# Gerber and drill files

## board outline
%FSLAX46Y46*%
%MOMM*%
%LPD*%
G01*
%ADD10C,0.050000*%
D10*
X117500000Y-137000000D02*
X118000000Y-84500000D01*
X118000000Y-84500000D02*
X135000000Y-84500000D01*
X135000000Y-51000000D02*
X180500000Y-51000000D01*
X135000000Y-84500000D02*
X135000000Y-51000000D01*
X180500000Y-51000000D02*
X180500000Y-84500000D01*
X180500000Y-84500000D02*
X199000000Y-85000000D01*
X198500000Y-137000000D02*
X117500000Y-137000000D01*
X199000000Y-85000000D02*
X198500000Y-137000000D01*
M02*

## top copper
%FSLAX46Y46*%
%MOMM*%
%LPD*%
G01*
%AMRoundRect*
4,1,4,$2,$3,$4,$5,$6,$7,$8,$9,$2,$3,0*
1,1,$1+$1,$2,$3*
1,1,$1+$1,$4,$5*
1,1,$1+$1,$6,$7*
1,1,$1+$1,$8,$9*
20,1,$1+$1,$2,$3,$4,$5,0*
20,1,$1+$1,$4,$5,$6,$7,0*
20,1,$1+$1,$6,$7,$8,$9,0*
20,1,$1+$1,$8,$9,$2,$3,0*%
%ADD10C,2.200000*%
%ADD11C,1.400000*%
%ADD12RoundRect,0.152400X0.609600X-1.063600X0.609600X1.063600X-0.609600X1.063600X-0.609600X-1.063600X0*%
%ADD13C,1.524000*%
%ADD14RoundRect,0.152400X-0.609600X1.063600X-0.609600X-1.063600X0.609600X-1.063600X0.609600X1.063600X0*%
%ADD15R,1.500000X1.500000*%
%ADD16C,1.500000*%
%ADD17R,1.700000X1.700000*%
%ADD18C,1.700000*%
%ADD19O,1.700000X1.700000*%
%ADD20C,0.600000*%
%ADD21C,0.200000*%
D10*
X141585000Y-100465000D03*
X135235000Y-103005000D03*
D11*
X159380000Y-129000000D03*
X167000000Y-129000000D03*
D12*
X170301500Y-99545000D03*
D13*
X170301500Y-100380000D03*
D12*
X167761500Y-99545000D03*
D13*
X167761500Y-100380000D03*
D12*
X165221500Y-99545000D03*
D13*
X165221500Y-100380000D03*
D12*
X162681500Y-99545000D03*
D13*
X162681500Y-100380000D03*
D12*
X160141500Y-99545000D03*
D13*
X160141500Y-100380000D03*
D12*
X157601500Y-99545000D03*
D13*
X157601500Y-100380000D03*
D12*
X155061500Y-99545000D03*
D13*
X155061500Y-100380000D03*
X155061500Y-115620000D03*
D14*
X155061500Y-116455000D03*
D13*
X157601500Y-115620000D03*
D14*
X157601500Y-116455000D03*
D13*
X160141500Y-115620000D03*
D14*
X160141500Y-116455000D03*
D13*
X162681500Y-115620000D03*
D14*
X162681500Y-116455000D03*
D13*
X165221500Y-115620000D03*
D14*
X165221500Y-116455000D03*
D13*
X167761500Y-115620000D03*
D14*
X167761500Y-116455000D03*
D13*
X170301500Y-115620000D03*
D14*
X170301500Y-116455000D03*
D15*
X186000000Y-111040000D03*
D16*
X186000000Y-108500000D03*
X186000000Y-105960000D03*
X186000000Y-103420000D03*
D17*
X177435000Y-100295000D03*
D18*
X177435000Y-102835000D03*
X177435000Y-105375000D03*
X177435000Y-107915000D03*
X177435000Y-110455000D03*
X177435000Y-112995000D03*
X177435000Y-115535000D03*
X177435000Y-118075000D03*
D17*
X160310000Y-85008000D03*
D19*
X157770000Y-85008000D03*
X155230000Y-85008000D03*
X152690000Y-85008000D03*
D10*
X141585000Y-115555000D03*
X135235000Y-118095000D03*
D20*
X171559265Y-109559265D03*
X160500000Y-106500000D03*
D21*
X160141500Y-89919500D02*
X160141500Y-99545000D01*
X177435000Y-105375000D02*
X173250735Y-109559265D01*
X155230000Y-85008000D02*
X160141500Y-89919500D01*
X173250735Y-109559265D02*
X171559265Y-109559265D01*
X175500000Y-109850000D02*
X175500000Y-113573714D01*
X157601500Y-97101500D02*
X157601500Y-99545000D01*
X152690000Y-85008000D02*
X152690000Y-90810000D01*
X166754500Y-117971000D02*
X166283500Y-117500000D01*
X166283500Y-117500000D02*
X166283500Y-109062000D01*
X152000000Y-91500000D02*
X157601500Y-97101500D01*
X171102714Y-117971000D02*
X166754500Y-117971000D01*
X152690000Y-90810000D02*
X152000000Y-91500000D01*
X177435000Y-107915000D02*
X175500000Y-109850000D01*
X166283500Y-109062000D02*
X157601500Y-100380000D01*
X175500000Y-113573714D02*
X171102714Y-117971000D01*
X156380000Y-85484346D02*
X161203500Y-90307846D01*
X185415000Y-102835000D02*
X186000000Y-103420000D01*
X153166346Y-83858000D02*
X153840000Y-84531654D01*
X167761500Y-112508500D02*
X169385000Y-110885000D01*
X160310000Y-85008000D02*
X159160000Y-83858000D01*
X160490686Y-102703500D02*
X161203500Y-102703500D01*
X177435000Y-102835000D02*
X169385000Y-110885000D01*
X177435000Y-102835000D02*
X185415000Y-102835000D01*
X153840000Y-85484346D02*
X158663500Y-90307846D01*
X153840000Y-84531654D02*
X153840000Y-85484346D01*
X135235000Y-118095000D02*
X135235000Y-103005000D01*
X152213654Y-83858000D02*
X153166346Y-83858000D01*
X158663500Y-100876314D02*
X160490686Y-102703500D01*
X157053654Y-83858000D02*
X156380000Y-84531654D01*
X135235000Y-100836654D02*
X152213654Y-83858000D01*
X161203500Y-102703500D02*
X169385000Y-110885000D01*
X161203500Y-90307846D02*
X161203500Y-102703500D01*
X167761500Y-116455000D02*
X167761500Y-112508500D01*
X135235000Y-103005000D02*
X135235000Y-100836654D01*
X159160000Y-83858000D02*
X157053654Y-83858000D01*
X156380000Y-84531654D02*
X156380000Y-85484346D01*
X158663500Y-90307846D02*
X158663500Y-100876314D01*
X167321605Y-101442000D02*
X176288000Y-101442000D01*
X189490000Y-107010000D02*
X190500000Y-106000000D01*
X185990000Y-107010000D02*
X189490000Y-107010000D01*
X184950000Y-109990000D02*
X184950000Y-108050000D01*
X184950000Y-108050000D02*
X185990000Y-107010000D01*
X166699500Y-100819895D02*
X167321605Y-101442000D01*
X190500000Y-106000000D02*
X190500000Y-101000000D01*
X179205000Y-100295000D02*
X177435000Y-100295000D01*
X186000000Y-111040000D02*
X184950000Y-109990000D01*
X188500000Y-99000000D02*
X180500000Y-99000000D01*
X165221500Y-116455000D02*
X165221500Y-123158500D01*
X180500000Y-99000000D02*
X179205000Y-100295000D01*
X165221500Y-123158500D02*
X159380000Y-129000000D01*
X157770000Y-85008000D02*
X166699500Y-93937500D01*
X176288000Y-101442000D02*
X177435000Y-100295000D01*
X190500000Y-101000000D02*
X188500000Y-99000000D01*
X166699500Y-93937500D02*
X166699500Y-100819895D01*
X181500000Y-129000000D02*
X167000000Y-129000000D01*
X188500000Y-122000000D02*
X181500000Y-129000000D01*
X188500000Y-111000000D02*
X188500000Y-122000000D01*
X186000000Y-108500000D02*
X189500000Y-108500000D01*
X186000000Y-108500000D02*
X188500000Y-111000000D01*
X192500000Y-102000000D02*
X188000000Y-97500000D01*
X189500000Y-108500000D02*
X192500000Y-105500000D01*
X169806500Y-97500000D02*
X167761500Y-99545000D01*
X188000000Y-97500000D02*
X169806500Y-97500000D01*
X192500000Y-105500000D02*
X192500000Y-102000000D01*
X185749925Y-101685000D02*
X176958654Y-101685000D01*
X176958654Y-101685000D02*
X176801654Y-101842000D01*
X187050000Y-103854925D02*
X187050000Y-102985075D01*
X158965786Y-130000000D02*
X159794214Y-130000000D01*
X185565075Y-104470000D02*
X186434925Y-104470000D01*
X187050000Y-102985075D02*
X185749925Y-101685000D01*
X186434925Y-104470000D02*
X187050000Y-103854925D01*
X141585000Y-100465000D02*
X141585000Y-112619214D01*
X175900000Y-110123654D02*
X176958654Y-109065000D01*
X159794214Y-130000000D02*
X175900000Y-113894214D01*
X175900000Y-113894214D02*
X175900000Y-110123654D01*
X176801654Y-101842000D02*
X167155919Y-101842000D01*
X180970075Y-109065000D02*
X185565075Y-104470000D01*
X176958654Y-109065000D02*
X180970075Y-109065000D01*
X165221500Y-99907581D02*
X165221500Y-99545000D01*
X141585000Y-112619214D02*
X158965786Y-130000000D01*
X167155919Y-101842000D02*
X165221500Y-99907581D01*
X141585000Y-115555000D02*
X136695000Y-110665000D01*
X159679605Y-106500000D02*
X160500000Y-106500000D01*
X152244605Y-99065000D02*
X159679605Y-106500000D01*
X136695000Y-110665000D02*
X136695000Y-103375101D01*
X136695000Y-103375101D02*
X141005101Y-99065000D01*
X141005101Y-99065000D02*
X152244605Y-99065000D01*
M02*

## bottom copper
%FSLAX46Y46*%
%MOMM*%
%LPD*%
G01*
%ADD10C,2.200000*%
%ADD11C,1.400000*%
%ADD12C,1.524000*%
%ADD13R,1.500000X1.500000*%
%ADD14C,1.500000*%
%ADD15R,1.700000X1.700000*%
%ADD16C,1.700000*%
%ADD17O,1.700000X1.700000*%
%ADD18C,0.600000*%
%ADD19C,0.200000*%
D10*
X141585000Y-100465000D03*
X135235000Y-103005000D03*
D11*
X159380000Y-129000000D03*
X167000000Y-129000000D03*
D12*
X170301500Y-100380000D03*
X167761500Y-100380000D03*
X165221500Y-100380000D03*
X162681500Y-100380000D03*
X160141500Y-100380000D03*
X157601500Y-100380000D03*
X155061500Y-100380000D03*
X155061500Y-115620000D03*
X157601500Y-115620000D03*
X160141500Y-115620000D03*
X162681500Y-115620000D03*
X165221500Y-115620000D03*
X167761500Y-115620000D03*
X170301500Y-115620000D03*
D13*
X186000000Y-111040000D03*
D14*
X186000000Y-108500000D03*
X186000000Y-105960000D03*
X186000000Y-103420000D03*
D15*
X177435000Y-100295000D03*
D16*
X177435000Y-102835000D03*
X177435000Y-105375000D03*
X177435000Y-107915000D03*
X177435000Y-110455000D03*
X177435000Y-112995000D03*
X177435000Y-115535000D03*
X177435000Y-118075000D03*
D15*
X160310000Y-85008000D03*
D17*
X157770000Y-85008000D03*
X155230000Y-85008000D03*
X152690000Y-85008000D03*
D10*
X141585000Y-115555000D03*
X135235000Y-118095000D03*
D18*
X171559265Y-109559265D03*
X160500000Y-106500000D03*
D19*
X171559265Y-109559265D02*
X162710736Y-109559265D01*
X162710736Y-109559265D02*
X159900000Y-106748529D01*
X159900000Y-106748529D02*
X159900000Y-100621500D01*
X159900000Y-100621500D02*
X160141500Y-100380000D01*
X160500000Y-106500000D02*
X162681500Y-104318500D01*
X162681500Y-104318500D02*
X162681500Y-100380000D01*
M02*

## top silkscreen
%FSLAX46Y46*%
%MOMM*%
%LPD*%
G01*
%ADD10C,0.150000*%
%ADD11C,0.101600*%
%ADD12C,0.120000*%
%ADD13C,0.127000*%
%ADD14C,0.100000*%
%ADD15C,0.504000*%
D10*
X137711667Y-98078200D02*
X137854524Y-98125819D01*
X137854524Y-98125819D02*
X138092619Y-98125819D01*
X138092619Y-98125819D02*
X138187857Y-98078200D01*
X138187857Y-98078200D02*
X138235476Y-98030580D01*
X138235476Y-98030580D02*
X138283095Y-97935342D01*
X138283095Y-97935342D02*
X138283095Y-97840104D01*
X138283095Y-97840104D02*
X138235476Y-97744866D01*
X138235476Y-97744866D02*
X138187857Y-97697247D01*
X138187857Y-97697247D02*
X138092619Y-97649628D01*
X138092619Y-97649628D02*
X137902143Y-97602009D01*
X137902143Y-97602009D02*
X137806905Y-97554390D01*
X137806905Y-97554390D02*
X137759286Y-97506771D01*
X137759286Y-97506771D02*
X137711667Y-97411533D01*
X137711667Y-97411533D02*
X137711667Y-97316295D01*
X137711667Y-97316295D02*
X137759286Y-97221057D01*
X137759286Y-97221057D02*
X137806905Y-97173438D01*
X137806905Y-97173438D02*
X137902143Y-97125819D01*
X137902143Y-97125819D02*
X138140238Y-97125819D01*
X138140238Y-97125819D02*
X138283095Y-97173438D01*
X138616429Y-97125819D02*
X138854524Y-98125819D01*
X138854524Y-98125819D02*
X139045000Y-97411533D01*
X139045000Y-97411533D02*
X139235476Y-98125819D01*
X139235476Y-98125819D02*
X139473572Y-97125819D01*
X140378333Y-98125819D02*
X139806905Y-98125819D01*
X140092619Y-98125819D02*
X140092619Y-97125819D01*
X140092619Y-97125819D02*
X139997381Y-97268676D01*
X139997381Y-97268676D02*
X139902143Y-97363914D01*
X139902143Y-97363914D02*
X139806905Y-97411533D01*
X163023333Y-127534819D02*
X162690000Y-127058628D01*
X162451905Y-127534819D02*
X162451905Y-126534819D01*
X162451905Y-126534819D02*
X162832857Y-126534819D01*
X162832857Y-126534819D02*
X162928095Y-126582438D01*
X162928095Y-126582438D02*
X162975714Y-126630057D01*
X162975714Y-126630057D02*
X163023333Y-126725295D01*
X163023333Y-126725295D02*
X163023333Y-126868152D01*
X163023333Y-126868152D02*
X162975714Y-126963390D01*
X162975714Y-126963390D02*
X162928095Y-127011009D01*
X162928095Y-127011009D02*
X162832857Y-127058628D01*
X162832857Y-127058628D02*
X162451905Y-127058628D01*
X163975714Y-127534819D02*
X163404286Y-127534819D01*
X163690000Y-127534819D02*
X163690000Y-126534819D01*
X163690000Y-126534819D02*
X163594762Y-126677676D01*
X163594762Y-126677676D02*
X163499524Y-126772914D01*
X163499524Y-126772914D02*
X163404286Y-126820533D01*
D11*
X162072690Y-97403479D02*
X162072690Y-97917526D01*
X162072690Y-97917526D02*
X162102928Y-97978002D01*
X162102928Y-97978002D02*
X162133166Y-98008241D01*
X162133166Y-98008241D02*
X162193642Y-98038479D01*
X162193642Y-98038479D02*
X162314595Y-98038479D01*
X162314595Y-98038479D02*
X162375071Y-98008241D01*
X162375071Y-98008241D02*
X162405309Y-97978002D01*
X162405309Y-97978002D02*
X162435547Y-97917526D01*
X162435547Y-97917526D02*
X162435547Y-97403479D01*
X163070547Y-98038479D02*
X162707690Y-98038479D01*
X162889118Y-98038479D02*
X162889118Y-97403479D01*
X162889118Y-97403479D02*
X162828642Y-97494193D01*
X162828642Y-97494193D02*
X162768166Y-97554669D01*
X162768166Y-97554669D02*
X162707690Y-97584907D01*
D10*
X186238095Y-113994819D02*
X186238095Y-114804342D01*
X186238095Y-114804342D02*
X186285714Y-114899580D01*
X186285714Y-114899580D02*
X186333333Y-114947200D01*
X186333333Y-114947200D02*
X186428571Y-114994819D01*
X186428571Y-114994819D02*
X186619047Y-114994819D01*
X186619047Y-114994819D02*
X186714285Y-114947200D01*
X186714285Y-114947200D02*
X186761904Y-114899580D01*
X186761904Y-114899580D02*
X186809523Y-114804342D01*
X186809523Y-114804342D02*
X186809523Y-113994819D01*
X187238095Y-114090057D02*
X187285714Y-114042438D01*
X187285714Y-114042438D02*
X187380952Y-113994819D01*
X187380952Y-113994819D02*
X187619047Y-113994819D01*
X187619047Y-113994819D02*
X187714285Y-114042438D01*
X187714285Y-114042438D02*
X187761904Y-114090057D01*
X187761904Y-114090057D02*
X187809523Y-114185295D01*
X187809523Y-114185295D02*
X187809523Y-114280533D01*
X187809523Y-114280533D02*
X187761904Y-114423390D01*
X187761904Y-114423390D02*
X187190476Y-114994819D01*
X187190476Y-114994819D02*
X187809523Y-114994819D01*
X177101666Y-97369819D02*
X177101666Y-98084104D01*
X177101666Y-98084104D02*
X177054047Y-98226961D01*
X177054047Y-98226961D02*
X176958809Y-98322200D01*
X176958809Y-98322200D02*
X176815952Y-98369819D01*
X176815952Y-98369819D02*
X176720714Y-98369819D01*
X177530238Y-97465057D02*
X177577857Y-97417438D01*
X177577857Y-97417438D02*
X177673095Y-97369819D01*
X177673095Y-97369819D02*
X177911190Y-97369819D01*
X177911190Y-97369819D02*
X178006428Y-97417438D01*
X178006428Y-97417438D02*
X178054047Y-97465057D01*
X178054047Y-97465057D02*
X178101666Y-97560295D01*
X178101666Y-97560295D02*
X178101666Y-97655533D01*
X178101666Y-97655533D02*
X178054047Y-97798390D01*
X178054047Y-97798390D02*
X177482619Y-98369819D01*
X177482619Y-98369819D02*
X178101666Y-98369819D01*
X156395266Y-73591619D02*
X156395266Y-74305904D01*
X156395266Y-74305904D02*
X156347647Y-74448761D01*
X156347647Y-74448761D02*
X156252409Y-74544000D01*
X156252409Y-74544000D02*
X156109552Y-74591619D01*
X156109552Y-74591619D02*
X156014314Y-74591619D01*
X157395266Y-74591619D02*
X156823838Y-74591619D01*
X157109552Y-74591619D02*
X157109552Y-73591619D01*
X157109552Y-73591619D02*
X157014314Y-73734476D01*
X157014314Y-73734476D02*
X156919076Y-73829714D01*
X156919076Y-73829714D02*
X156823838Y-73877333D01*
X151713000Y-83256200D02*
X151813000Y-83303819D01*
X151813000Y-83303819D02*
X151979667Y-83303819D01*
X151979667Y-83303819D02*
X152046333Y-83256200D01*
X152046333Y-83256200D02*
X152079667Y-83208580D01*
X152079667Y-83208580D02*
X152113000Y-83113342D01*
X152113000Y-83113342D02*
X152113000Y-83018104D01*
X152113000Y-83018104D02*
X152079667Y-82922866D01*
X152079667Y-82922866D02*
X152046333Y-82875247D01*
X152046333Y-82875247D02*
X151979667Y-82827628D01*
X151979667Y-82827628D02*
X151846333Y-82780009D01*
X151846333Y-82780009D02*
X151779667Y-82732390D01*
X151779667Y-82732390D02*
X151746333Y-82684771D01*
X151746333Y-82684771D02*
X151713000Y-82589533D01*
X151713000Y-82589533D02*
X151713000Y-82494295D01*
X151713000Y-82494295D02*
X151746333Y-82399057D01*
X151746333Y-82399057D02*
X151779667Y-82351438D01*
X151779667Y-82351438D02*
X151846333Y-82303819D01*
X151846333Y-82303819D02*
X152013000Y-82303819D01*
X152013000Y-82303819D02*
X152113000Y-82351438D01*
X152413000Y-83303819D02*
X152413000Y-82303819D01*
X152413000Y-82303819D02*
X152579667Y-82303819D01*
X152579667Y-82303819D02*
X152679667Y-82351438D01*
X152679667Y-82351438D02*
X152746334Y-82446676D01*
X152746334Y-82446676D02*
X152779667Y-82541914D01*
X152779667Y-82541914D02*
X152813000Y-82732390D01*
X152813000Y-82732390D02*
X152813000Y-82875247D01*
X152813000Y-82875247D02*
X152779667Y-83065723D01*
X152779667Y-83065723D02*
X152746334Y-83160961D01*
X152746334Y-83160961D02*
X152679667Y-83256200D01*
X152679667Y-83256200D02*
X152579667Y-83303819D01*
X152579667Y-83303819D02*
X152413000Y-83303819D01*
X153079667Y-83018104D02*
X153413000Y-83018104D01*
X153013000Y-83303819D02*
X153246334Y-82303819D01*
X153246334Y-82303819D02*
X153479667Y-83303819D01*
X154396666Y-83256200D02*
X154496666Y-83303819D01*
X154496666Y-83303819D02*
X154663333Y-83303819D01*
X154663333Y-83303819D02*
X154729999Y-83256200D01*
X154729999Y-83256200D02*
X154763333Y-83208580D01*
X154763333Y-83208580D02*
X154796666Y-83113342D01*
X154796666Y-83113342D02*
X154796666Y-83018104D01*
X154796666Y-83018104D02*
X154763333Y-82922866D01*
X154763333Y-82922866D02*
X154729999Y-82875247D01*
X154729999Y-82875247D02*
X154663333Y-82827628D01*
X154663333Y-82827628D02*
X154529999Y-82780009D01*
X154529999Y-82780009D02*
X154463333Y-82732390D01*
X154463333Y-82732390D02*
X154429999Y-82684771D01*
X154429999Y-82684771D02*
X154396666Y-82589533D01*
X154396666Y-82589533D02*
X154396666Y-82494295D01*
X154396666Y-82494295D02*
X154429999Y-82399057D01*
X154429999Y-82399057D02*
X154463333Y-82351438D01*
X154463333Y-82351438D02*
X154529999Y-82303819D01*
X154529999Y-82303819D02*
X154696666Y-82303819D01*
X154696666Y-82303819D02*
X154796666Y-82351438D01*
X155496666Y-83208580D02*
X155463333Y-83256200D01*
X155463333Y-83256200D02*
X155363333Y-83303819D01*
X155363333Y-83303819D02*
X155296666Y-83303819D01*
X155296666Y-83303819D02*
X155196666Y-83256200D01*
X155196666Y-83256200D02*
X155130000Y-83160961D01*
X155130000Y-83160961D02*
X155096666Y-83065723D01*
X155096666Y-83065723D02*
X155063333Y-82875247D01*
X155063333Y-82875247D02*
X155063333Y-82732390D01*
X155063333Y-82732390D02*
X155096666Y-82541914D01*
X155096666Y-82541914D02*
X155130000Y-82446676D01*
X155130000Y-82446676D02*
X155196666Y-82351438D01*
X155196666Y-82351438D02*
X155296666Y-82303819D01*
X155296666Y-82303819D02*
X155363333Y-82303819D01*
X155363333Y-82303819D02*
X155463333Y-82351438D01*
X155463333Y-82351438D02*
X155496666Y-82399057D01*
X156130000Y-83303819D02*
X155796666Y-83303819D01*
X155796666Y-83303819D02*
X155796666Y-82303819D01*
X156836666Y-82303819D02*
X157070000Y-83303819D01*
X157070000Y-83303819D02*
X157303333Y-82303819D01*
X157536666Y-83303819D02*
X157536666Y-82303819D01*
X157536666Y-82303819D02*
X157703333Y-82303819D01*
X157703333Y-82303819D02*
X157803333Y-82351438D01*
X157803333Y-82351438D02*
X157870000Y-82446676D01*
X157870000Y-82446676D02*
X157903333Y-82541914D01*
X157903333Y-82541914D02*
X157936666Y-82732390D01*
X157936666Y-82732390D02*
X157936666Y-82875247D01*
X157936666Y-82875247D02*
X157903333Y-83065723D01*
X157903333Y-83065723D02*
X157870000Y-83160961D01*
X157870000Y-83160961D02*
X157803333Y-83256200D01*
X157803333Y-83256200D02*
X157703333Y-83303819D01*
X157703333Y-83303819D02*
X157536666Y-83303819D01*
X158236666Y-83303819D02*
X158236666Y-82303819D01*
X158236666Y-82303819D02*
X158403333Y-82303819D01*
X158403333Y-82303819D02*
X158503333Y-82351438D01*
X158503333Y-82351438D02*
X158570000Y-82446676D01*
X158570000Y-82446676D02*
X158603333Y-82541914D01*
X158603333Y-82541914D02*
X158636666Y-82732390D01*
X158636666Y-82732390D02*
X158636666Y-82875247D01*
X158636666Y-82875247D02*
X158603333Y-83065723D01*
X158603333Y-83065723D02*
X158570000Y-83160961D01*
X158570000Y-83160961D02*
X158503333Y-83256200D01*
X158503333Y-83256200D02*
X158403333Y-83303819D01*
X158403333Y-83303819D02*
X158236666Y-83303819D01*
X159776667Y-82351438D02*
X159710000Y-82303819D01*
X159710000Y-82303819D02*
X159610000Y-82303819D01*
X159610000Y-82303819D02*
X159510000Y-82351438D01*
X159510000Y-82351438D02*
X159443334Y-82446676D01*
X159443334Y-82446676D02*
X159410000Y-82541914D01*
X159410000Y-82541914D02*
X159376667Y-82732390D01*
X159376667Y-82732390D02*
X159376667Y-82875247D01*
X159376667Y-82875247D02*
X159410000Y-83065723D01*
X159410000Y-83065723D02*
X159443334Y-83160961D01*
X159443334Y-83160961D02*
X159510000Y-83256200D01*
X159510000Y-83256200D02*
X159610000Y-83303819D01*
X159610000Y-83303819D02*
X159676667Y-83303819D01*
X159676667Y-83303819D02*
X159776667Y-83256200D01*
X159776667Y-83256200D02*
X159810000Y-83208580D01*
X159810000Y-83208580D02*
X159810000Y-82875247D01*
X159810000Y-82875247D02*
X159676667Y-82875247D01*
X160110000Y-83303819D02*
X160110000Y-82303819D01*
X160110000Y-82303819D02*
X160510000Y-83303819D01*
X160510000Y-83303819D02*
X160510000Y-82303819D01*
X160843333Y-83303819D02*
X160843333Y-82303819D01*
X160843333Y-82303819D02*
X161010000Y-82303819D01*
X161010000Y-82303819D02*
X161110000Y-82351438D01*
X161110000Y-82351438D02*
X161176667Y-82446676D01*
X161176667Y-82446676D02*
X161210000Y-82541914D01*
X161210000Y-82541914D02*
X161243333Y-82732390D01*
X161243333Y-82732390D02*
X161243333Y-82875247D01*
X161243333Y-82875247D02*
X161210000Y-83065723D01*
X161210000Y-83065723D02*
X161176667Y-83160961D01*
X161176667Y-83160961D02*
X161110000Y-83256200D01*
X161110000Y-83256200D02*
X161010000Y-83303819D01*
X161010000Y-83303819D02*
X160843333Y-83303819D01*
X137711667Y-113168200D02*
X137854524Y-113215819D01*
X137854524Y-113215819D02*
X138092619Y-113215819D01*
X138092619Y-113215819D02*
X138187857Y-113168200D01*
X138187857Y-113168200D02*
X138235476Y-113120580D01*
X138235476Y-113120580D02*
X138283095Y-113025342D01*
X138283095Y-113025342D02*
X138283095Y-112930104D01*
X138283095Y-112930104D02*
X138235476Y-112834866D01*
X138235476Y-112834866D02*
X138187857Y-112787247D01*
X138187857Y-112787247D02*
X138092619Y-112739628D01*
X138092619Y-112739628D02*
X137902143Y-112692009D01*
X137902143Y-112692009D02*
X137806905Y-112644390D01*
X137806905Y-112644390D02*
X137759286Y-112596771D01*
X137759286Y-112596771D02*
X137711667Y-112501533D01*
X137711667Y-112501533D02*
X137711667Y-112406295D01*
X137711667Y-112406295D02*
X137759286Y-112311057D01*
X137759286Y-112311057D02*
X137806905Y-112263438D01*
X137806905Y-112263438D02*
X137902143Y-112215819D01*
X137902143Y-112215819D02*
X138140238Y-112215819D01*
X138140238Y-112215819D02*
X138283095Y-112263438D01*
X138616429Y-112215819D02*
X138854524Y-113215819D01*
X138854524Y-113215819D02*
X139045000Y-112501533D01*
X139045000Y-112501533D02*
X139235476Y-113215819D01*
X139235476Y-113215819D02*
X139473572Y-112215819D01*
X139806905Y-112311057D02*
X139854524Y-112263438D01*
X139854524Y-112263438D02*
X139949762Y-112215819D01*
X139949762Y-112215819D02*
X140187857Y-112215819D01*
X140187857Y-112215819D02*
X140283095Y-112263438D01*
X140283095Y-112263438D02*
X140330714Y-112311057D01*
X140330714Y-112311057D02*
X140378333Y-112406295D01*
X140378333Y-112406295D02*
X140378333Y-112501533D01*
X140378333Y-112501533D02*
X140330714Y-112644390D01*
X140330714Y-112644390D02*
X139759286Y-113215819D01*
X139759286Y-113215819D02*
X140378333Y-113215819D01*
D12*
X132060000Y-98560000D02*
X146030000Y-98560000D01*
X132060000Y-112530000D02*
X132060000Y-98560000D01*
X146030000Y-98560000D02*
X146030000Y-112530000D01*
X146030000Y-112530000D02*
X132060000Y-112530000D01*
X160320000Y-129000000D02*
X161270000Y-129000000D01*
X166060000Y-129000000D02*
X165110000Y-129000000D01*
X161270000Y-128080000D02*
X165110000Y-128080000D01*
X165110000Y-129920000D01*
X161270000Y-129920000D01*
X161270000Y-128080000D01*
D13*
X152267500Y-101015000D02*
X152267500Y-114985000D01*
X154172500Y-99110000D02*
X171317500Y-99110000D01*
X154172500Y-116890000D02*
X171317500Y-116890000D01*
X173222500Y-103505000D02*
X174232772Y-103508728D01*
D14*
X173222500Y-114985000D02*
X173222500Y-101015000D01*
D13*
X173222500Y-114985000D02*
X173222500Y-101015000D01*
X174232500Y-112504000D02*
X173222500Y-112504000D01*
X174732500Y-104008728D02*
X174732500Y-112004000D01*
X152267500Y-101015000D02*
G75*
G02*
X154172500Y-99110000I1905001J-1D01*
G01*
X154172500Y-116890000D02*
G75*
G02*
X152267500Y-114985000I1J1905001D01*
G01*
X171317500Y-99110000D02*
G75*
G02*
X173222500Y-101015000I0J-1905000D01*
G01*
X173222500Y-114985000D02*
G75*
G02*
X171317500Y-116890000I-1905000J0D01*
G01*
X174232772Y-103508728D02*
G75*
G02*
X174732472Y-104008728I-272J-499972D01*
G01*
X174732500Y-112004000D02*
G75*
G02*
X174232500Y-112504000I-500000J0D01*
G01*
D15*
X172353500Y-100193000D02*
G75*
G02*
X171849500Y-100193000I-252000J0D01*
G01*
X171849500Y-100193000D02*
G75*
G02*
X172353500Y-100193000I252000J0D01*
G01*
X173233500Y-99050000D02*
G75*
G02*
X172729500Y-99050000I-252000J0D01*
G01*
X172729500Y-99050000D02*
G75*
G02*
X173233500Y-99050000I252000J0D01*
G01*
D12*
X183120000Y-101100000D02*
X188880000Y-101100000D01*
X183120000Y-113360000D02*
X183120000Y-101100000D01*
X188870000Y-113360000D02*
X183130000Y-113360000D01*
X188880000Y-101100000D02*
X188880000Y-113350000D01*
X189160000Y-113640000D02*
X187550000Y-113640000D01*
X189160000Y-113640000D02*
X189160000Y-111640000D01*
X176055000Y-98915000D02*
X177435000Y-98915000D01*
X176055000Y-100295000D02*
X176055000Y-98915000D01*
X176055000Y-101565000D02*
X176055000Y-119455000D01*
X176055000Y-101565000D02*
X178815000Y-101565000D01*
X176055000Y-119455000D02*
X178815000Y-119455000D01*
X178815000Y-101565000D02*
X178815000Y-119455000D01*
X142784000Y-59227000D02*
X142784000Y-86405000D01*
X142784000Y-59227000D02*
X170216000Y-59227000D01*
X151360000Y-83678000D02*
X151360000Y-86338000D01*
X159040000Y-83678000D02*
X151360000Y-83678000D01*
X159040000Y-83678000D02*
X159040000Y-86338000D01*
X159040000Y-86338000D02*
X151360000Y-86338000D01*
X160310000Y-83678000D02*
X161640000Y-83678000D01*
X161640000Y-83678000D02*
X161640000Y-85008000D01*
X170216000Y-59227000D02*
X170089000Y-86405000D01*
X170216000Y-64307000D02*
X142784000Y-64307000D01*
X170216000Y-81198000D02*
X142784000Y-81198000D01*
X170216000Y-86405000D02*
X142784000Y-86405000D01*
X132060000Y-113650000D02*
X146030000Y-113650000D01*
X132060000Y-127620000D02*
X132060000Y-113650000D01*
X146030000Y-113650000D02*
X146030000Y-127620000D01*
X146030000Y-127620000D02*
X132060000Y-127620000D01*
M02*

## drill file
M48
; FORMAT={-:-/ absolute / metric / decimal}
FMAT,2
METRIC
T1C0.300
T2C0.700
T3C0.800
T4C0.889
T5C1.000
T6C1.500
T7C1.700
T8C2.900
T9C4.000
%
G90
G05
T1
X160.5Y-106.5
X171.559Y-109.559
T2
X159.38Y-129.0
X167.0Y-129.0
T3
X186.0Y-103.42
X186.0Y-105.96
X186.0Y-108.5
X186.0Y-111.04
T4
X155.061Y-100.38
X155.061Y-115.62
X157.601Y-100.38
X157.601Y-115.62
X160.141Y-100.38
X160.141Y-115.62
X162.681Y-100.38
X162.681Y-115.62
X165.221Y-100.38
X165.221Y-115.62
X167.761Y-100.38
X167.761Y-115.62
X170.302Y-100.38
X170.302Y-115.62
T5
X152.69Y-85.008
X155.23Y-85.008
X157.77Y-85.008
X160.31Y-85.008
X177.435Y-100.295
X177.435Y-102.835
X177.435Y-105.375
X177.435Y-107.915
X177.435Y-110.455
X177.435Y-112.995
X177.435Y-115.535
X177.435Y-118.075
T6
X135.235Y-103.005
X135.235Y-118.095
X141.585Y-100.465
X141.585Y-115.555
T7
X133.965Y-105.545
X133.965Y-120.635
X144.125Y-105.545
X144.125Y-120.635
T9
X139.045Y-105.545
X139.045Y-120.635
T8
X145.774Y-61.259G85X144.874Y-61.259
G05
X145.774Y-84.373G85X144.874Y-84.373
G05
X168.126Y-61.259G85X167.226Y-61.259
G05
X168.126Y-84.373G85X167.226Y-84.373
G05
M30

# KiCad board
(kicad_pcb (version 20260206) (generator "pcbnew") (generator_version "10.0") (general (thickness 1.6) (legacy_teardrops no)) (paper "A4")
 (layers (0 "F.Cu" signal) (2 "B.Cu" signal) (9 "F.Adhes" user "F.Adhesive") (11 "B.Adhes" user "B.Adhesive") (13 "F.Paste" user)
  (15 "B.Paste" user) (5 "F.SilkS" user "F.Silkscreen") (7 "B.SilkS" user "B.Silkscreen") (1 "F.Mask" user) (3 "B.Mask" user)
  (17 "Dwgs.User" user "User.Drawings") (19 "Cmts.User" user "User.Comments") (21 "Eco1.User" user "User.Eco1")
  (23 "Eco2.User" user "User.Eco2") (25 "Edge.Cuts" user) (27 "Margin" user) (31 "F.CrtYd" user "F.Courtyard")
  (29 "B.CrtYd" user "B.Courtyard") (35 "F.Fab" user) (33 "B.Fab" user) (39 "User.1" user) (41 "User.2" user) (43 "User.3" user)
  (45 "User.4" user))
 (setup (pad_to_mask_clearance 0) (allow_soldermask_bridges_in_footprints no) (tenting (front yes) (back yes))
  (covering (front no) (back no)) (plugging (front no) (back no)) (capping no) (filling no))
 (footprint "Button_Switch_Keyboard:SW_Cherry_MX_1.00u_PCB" (layer "F.Cu") (at 141.585 100.465)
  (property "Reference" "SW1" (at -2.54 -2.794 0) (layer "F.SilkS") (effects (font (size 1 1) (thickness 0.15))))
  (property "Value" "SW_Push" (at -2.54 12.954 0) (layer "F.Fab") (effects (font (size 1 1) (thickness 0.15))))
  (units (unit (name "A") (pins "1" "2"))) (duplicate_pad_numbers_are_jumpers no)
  (fp_line (start -9.525 -1.905) (end 4.445 -1.905) (stroke (width 0.12) (type solid)) (layer "F.SilkS"))
  (fp_line (start -9.525 12.065) (end -9.525 -1.905) (stroke (width 0.12) (type solid)) (layer "F.SilkS"))
  (fp_line (start 4.445 -1.905) (end 4.445 12.065) (stroke (width 0.12) (type solid)) (layer "F.SilkS"))
  (fp_line (start 4.445 12.065) (end -9.525 12.065) (stroke (width 0.12) (type solid)) (layer "F.SilkS"))
  (pad "" np_thru_hole circle (at -7.62 5.08) (size 1.7 1.7) (drill 1.7) (layers "*.Cu" "*.Mask"))
  (pad "" np_thru_hole circle (at -2.54 5.08) (size 4 4) (drill 4) (layers "*.Cu" "*.Mask"))
  (pad "" np_thru_hole circle (at 2.54 5.08) (size 1.7 1.7) (drill 1.7) (layers "*.Cu" "*.Mask"))
  (pad "1" thru_hole circle (at 0 0) (size 2.2 2.2) (drill 1.5) (layers "*.Cu" "*.Mask") (remove_unused_layers no) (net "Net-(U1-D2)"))
  (pad "2" thru_hole circle (at -6.35 2.54) (size 2.2 2.2) (drill 1.5) (layers "*.Cu" "*.Mask") (remove_unused_layers no) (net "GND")))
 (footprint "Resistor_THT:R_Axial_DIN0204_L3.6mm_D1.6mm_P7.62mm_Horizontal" (layer "F.Cu") (at 159.38 129)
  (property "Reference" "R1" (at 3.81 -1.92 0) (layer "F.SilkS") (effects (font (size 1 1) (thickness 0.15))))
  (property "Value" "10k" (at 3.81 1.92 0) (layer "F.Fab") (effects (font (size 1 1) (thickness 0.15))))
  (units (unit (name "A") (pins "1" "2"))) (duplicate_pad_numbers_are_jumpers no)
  (fp_line (start 0.94 0) (end 1.89 0) (stroke (width 0.12) (type solid)) (layer "F.SilkS"))
  (fp_line (start 6.68 0) (end 5.73 0) (stroke (width 0.12) (type solid)) (layer "F.SilkS"))
  (fp_rect (start 1.89 -0.92) (end 5.73 0.92) (stroke (width 0.12) (type solid)) (fill no) (layer "F.SilkS"))
  (pad "1" thru_hole circle (at 0 0) (size 1.4 1.4) (drill 0.7) (layers "*.Cu" "*.Mask") (remove_unused_layers no) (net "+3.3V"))
  (pad "2" thru_hole circle (at 7.62 0) (size 1.4 1.4) (drill 0.7) (layers "*.Cu" "*.Mask") (remove_unused_layers no) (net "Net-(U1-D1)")))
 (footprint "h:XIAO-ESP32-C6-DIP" (layer "F.Cu") (at 162.6815 108)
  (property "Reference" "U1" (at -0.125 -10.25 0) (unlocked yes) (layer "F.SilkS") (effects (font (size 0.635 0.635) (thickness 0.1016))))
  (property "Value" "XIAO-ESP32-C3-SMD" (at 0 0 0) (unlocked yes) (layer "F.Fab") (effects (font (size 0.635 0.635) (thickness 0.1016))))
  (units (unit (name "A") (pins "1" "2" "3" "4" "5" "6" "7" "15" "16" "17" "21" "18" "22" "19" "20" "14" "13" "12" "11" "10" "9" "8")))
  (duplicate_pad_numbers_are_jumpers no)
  (fp_line (start -10.414 -6.985) (end -10.414 6.985) (stroke (width 0.127) (type solid)) (layer "F.SilkS"))
  (fp_line (start -8.509 -8.89) (end 8.636 -8.89) (stroke (width 0.127) (type solid)) (layer "F.SilkS"))
  (fp_line (start -8.509 8.89) (end 8.636 8.89) (stroke (width 0.127) (type solid)) (layer "F.SilkS"))
  (fp_line (start 10.541 -4.495) (end 11.551272 -4.491272) (stroke (width 0.127) (type solid)) (layer "F.SilkS"))
  (fp_line (start 10.541 6.985) (end 10.541 -6.985) (stroke (width 0.1) (type solid)) (layer "F.SilkS"))
  (fp_line (start 10.541 6.985) (end 10.541 -6.985) (stroke (width 0.127) (type solid)) (layer "F.SilkS"))
  (fp_line (start 11.551 4.504) (end 10.541 4.504) (stroke (width 0.127) (type solid)) (layer "F.SilkS"))
  (fp_line (start 12.051 -3.991272) (end 12.051 4.004) (stroke (width 0.127) (type solid)) (layer "F.SilkS"))
  (fp_arc (start -10.414 -6.985) (mid -9.856038 -8.332038) (end -8.509 -8.89) (stroke (width 0.127) (type solid)) (layer "F.SilkS"))
  (fp_arc (start -8.509 8.89) (mid -9.856038 8.332038) (end -10.414 6.985) (stroke (width 0.127) (type solid)) (layer "F.SilkS"))
  (fp_arc (start 8.636 -8.89) (mid 9.983038 -8.332038) (end 10.541 -6.985) (stroke (width 0.127) (type solid)) (layer "F.SilkS"))
  (fp_arc (start 10.541 6.985) (mid 9.983038 8.332038) (end 8.636 8.89) (stroke (width 0.127) (type solid)) (layer "F.SilkS"))
  (fp_arc (start 11.551272 -4.491272) (mid 11.904644 -4.344724) (end 12.051 -3.991272) (stroke (width 0.127) (type default))
   (layer "F.SilkS"))
  (fp_arc (start 12.051 4.004) (mid 11.904553 4.357553) (end 11.551 4.504) (stroke (width 0.127) (type default)) (layer "F.SilkS"))
  (fp_circle (center 9.42 -7.807) (end 9.674 -7.807) (stroke (width 0.5) (type solid)) (fill yes) (layer "F.SilkS"))
  (fp_circle (center 10.3 -8.95) (end 10.554 -8.95) (stroke (width 0.5) (type solid)) (fill yes) (layer "F.SilkS"))
  (pad "1" smd roundrect (at 7.62 -8.455 90) (size 2.432 1.524) (layers "F.Cu" "F.Mask") (roundrect_rratio 0.1)
   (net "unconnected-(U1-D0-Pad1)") (thermal_bridge_angle 45))
  (pad "1" thru_hole circle (at 7.62 -7.62 90) (size 1.524 1.524) (drill 0.889) (layers "*.Cu" "*.Mask") (remove_unused_layers no)
   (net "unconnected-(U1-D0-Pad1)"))
  (pad "2" smd roundrect (at 5.08 -8.455 90) (size 2.432 1.524) (layers "F.Cu" "F.Mask") (roundrect_rratio 0.1) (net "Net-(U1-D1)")
   (thermal_bridge_angle 45))
  (pad "2" thru_hole circle (at 5.08 -7.62 90) (size 1.524 1.524) (drill 0.889) (layers "*.Cu" "*.Mask") (remove_unused_layers no)
   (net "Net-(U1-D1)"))
  (pad "3" smd roundrect (at 2.54 -8.455 90) (size 2.432 1.524) (layers "F.Cu" "F.Mask") (roundrect_rratio 0.1) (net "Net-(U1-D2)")
   (thermal_bridge_angle 45))
  (pad "3" thru_hole circle (at 2.54 -7.62 90) (size 1.524 1.524) (drill 0.889) (layers "*.Cu" "*.Mask") (remove_unused_layers no)
   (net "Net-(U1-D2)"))
  (pad "4" smd roundrect (at 0 -8.455 90) (size 2.432 1.524) (layers "F.Cu" "F.Mask") (roundrect_rratio 0.1) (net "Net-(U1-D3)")
   (thermal_bridge_angle 45))
  (pad "4" thru_hole circle (at 0 -7.62 90) (size 1.524 1.524) (drill 0.889) (layers "*.Cu" "*.Mask") (remove_unused_layers no)
   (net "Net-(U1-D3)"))
  (pad "5" smd roundrect (at -2.54 -8.455 90) (size 2.432 1.524) (layers "F.Cu" "F.Mask") (roundrect_rratio 0.1) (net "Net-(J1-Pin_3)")
   (thermal_bridge_angle 45))
  (pad "5" thru_hole circle (at -2.54 -7.62 90) (size 1.524 1.524) (drill 0.889) (layers "*.Cu" "*.Mask") (remove_unused_layers no)
   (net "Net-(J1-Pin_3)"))
  (pad "6" smd roundrect (at -5.08 -8.455 90) (size 2.432 1.524) (layers "F.Cu" "F.Mask") (roundrect_rratio 0.1) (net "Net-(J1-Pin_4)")
   (thermal_bridge_angle 45))
  (pad "6" thru_hole circle (at -5.08 -7.62 90) (size 1.524 1.524) (drill 0.889) (layers "*.Cu" "*.Mask") (remove_unused_layers no)
   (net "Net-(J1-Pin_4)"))
  (pad "7" smd roundrect (at -7.62 -8.455 90) (size 2.432 1.524) (layers "F.Cu" "F.Mask") (roundrect_rratio 0.1)
   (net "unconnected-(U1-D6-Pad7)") (thermal_bridge_angle 45))
  (pad "7" thru_hole circle (at -7.62 -7.62 90) (size 1.524 1.524) (drill 0.889) (layers "*.Cu" "*.Mask") (remove_unused_layers no)
   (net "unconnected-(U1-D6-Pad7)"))
  (pad "8" thru_hole circle (at -7.62 7.62 270) (size 1.524 1.524) (drill 0.889) (layers "*.Cu" "*.Mask") (remove_unused_layers no)
   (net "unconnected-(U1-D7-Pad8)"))
  (pad "8" smd roundrect (at -7.62 8.455 270) (size 2.432 1.524) (layers "F.Cu" "F.Mask") (roundrect_rratio 0.1)
   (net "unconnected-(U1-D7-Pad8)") (thermal_bridge_angle 45))
  (pad "9" thru_hole circle (at -5.08 7.62 270) (size 1.524 1.524) (drill 0.889) (layers "*.Cu" "*.Mask") (remove_unused_layers no)
   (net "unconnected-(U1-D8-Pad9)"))
  (pad "9" smd roundrect (at -5.08 8.455 270) (size 2.432 1.524) (layers "F.Cu" "F.Mask") (roundrect_rratio 0.1)
   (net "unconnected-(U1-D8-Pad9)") (thermal_bridge_angle 45))
  (pad "10" thru_hole circle (at -2.54 7.62 270) (size 1.524 1.524) (drill 0.889) (layers "*.Cu" "*.Mask") (remove_unused_layers no)
   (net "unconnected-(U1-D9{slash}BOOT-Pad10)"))
  (pad "10" smd roundrect (at -2.54 8.455 270) (size 2.432 1.524) (layers "F.Cu" "F.Mask") (roundrect_rratio 0.1)
   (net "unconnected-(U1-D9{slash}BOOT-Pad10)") (thermal_bridge_angle 45))
  (pad "11" thru_hole circle (at 0 7.62 270) (size 1.524 1.524) (drill 0.889) (layers "*.Cu" "*.Mask") (remove_unused_layers no)
   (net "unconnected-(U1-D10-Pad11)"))
  (pad "11" smd roundrect (at 0 8.455 270) (size 2.432 1.524) (layers "F.Cu" "F.Mask") (roundrect_rratio 0.1)
   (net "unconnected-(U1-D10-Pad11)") (thermal_bridge_angle 45))
  (pad "12" thru_hole circle (at 2.54 7.62 270) (size 1.524 1.524) (drill 0.889) (layers "*.Cu" "*.Mask") (remove_unused_layers no)
   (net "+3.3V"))
  (pad "12" smd roundrect (at 2.54 8.455 270) (size 2.432 1.524) (layers "F.Cu" "F.Mask") (roundrect_rratio 0.1) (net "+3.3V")
   (thermal_bridge_angle 45))
  (pad "13" thru_hole circle (at 5.08 7.62 270) (size 1.524 1.524) (drill 0.889) (layers "*.Cu" "*.Mask") (remove_unused_layers no)
   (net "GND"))
  (pad "13" smd roundrect (at 5.08 8.455 270) (size 2.432 1.524) (layers "F.Cu" "F.Mask") (roundrect_rratio 0.1) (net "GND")
   (thermal_bridge_angle 45))
  (pad "14" thru_hole circle (at 7.62 7.62 270) (size 1.524 1.524) (drill 0.889) (layers "*.Cu" "*.Mask") (remove_unused_layers no)
   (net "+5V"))
  (pad "14" smd roundrect (at 7.62 8.455 270) (size 2.432 1.524) (layers "F.Cu" "F.Mask") (roundrect_rratio 0.1) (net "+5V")
   (thermal_bridge_angle 45)))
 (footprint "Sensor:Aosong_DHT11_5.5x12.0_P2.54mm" (layer "F.Cu") (at 186 111.04 180)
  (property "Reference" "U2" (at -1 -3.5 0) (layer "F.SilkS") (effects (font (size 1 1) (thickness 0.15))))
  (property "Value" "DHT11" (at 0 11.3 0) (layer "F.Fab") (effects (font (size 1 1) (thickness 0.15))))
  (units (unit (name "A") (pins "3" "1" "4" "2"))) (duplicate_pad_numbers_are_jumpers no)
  (fp_line (start 2.88 9.94) (end -2.88 9.94) (stroke (width 0.12) (type solid)) (layer "F.SilkS"))
  (fp_line (start 2.88 -2.32) (end 2.88 9.94) (stroke (width 0.12) (type solid)) (layer "F.SilkS"))
  (fp_line (start -2.87 -2.32) (end 2.87 -2.32) (stroke (width 0.12) (type solid)) (layer "F.SilkS"))
  (fp_line (start -2.88 9.94) (end -2.88 -2.31) (stroke (width 0.12) (type solid)) (layer "F.SilkS"))
  (fp_line (start -3.16 -2.6) (end -1.55 -2.6) (stroke (width 0.12) (type solid)) (layer "F.SilkS"))
  (fp_line (start -3.16 -2.6) (end -3.16 -0.6) (stroke (width 0.12) (type solid)) (layer "F.SilkS"))
  (pad "1" thru_hole rect (at 0 0 180) (size 1.5 1.5) (drill 0.8) (layers "*.Cu" "*.Mask") (remove_unused_layers no) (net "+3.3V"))
  (pad "2" thru_hole circle (at 0 2.54 180) (size 1.5 1.5) (drill 0.8) (layers "*.Cu" "*.Mask") (remove_unused_layers no)
   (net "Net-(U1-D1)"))
  (pad "3" thru_hole circle (at 0 5.08 180) (size 1.5 1.5) (drill 0.8) (layers "*.Cu" "*.Mask") (remove_unused_layers no)
   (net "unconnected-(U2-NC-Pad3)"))
  (pad "4" thru_hole circle (at 0 7.62 180) (size 1.5 1.5) (drill 0.8) (layers "*.Cu" "*.Mask") (remove_unused_layers no) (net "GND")))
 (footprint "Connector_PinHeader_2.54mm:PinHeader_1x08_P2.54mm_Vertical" (layer "F.Cu") (at 177.435 100.295)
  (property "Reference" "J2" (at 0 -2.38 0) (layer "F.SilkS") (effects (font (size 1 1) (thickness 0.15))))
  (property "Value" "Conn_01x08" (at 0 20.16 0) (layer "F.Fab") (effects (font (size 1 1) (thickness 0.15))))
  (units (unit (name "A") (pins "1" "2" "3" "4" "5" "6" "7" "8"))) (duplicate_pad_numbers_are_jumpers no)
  (fp_line (start -1.38 -1.38) (end 0 -1.38) (stroke (width 0.12) (type solid)) (layer "F.SilkS"))
  (fp_line (start -1.38 0) (end -1.38 -1.38) (stroke (width 0.12) (type solid)) (layer "F.SilkS"))
  (fp_line (start -1.38 1.27) (end -1.38 19.16) (stroke (width 0.12) (type solid)) (layer "F.SilkS"))
  (fp_line (start -1.38 1.27) (end 1.38 1.27) (stroke (width 0.12) (type solid)) (layer "F.SilkS"))
  (fp_line (start -1.38 19.16) (end 1.38 19.16) (stroke (width 0.12) (type solid)) (layer "F.SilkS"))
  (fp_line (start 1.38 1.27) (end 1.38 19.16) (stroke (width 0.12) (type solid)) (layer "F.SilkS"))
  (pad "1" thru_hole rect (at 0 0) (size 1.7 1.7) (drill 1) (layers "*.Cu" "*.Mask") (remove_unused_layers no) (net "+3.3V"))
  (pad "2" thru_hole circle (at 0 2.54) (size 1.7 1.7) (drill 1) (layers "*.Cu" "*.Mask") (remove_unused_layers no) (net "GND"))
  (pad "3" thru_hole circle (at 0 5.08) (size 1.7 1.7) (drill 1) (layers "*.Cu" "*.Mask") (remove_unused_layers no) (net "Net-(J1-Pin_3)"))
  (pad "4" thru_hole circle (at 0 7.62) (size 1.7 1.7) (drill 1) (layers "*.Cu" "*.Mask") (remove_unused_layers no) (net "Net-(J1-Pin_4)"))
  (pad "5" thru_hole circle (at 0 10.16) (size 1.7 1.7) (drill 1) (layers "*.Cu" "*.Mask") (remove_unused_layers no)
   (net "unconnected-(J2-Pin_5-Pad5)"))
  (pad "6" thru_hole circle (at 0 12.7) (size 1.7 1.7) (drill 1) (layers "*.Cu" "*.Mask") (remove_unused_layers no)
   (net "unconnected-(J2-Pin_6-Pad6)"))
  (pad "7" thru_hole circle (at 0 15.24) (size 1.7 1.7) (drill 1) (layers "*.Cu" "*.Mask") (remove_unused_layers no)
   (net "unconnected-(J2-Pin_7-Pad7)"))
  (pad "8" thru_hole circle (at 0 17.78) (size 1.7 1.7) (drill 1) (layers "*.Cu" "*.Mask") (remove_unused_layers no)
   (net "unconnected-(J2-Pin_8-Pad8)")))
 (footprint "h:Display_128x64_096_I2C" (layer "F.Cu") (at 156.5 85.008 180)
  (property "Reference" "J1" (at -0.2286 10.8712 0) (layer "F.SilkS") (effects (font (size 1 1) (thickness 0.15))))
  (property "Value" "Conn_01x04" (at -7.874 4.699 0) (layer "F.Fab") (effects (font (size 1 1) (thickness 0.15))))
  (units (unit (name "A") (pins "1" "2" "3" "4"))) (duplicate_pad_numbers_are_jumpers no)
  (fp_line (start 13.716 25.781) (end 13.716 -1.397) (stroke (width 0.12) (type solid)) (layer "F.SilkS"))
  (fp_line (start 13.716 25.781) (end -13.716 25.781) (stroke (width 0.12) (type solid)) (layer "F.SilkS"))
  (fp_line (start 5.14 1.33) (end 5.14 -1.33) (stroke (width 0.12) (type solid)) (layer "F.SilkS"))
  (fp_line (start -2.54 1.33) (end 5.14 1.33) (stroke (width 0.12) (type solid)) (layer "F.SilkS"))
  (fp_line (start -2.54 1.33) (end -2.54 -1.33) (stroke (width 0.12) (type solid)) (layer "F.SilkS"))
  (fp_line (start -2.54 -1.33) (end 5.14 -1.33) (stroke (width 0.12) (type solid)) (layer "F.SilkS"))
  (fp_line (start -3.81 1.33) (end -5.14 1.33) (stroke (width 0.12) (type solid)) (layer "F.SilkS"))
  (fp_line (start -5.14 1.33) (end -5.14 0) (stroke (width 0.12) (type solid)) (layer "F.SilkS"))
  (fp_line (start -13.716 25.781) (end -13.589 -1.397) (stroke (width 0.12) (type solid)) (layer "F.SilkS"))
  (fp_line (start -13.716 20.701) (end 13.716 20.701) (stroke (width 0.12) (type solid)) (layer "F.SilkS"))
  (fp_line (start -13.716 3.81) (end 13.716 3.81) (stroke (width 0.12) (type solid)) (layer "F.SilkS"))
  (fp_line (start -13.716 -1.397) (end 13.716 -1.397) (stroke (width 0.12) (type solid)) (layer "F.SilkS"))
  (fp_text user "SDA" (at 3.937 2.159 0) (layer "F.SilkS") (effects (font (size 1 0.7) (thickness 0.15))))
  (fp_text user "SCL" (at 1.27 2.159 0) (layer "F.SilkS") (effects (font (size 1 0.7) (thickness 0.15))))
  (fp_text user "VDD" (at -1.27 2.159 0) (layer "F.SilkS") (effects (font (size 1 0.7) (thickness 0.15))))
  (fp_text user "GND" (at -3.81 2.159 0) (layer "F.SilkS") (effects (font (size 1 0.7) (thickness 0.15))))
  (pad "" np_thru_hole oval (at -11.176 0.635 180) (size 3.8 2.9) (drill oval 3.8 2.9) (layers "*.Cu" "*.Mask"))
  (pad "" np_thru_hole oval (at -11.176 23.749 180) (size 3.8 2.9) (drill oval 3.8 2.9) (layers "*.Cu" "*.Mask"))
  (pad "" np_thru_hole oval (at 11.176 0.635 180) (size 3.8 2.9) (drill oval 3.8 2.9) (layers "*.Cu" "*.Mask"))
  (pad "" np_thru_hole oval (at 11.176 23.749 180) (size 3.8 2.9) (drill oval 3.8 2.9) (layers "*.Cu" "*.Mask"))
  (pad "1" thru_hole rect (at -3.81 0 270) (size 1.7 1.7) (drill 1) (layers "*.Cu" "*.Mask") (remove_unused_layers no) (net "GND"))
  (pad "2" thru_hole oval (at -1.27 0 270) (size 1.7 1.7) (drill 1) (layers "*.Cu" "*.Mask") (remove_unused_layers no) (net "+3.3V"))
  (pad "3" thru_hole oval (at 1.27 0 270) (size 1.7 1.7) (drill 1) (layers "*.Cu" "*.Mask") (remove_unused_layers no) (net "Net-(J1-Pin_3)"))
  (pad "4" thru_hole oval (at 3.81 0 270) (size 1.7 1.7) (drill 1) (layers "*.Cu" "*.Mask") (remove_unused_layers no) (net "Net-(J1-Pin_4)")))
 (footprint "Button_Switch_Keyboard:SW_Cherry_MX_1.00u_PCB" (layer "F.Cu") (at 141.585 115.555)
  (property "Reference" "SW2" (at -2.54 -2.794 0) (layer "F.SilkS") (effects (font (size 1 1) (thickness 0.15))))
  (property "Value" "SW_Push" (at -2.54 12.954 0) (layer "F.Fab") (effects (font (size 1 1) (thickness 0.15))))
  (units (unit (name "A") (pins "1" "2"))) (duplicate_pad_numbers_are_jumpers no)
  (fp_line (start -9.525 -1.905) (end 4.445 -1.905) (stroke (width 0.12) (type solid)) (layer "F.SilkS"))
  (fp_line (start -9.525 12.065) (end -9.525 -1.905) (stroke (width 0.12) (type solid)) (layer "F.SilkS"))
  (fp_line (start 4.445 -1.905) (end 4.445 12.065) (stroke (width 0.12) (type solid)) (layer "F.SilkS"))
  (fp_line (start 4.445 12.065) (end -9.525 12.065) (stroke (width 0.12) (type solid)) (layer "F.SilkS"))
  (pad "" np_thru_hole circle (at -7.62 5.08) (size 1.7 1.7) (drill 1.7) (layers "*.Cu" "*.Mask"))
  (pad "" np_thru_hole circle (at -2.54 5.08) (size 4 4) (drill 4) (layers "*.Cu" "*.Mask"))
  (pad "" np_thru_hole circle (at 2.54 5.08) (size 1.7 1.7) (drill 1.7) (layers "*.Cu" "*.Mask"))
  (pad "1" thru_hole circle (at 0 0) (size 2.2 2.2) (drill 1.5) (layers "*.Cu" "*.Mask") (remove_unused_layers no) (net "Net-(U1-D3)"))
  (pad "2" thru_hole circle (at -6.35 2.54) (size 2.2 2.2) (drill 1.5) (layers "*.Cu" "*.Mask") (remove_unused_layers no) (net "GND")))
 (gr_line (start 117.5 137) (end 118 84.5) (stroke (width 0.05) (type default)) (layer "Edge.Cuts"))
 (gr_line (start 118 84.5) (end 135 84.5) (stroke (width 0.05) (type default)) (layer "Edge.Cuts"))
 (gr_line (start 135 51) (end 180.5 51) (stroke (width 0.05) (type default)) (layer "Edge.Cuts"))
 (gr_line (start 135 84.5) (end 135 51) (stroke (width 0.05) (type default)) (layer "Edge.Cuts"))
 (gr_line (start 180.5 51) (end 180.5 84.5) (stroke (width 0.05) (type default)) (layer "Edge.Cuts"))
 (gr_line (start 180.5 84.5) (end 199 85) (stroke (width 0.05) (type default)) (layer "Edge.Cuts"))
 (gr_line (start 198.5 137) (end 117.5 137) (stroke (width 0.05) (type default)) (layer "Edge.Cuts"))
 (gr_line (start 199 85) (end 198.5 137) (stroke (width 0.05) (type default)) (layer "Edge.Cuts"))
 (segment (start 160.1415 89.9195) (end 160.1415 99.545) (width 0.2) (layer "F.Cu") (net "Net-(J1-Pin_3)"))
 (segment (start 177.435 105.375) (end 173.250735 109.559265) (width 0.2) (layer "F.Cu") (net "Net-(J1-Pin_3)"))
 (segment (start 155.23 85.008) (end 160.1415 89.9195) (width 0.2) (layer "F.Cu") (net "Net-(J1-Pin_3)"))
 (segment (start 173.250735 109.559265) (end 171.559265 109.559265) (width 0.2) (layer "F.Cu") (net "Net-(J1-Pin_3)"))
 (via (at 171.559265 109.559265) (size 0.6) (drill 0.3) (layers "F.Cu" "B.Cu") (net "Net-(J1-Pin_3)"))
 (segment (start 171.559265 109.559265) (end 162.710736 109.559265) (width 0.2) (layer "B.Cu") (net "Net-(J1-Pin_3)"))
 (segment (start 162.710736 109.559265) (end 159.9 106.748529) (width 0.2) (layer "B.Cu") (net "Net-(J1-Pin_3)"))
 (segment (start 159.9 106.748529) (end 159.9 100.6215) (width 0.2) (layer "B.Cu") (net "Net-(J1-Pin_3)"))
 (segment (start 159.9 100.6215) (end 160.1415 100.38) (width 0.2) (layer "B.Cu") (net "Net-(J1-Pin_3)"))
 (segment (start 175.5 109.85) (end 175.5 113.573714) (width 0.2) (layer "F.Cu") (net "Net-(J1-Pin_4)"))
 (segment (start 157.6015 97.1015) (end 157.6015 99.545) (width 0.2) (layer "F.Cu") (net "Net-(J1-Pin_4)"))
 (segment (start 152.69 85.008) (end 152.69 90.81) (width 0.2) (layer "F.Cu") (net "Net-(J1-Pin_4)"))
 (segment (start 166.7545 117.971) (end 166.2835 117.5) (width 0.2) (layer "F.Cu") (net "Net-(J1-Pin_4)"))
 (segment (start 166.2835 117.5) (end 166.2835 109.062) (width 0.2) (layer "F.Cu") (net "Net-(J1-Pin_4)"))
 (segment (start 152 91.5) (end 157.6015 97.1015) (width 0.2) (layer "F.Cu") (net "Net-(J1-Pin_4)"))
 (segment (start 171.102714 117.971) (end 166.7545 117.971) (width 0.2) (layer "F.Cu") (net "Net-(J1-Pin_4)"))
 (segment (start 152.69 90.81) (end 152 91.5) (width 0.2) (layer "F.Cu") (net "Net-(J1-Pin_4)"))
 (segment (start 177.435 107.915) (end 175.5 109.85) (width 0.2) (layer "F.Cu") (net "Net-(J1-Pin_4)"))
 (segment (start 166.2835 109.062) (end 157.6015 100.38) (width 0.2) (layer "F.Cu") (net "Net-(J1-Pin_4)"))
 (segment (start 175.5 113.573714) (end 171.102714 117.971) (width 0.2) (layer "F.Cu") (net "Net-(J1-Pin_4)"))
 (segment (start 156.38 85.484346) (end 161.2035 90.307846) (width 0.2) (layer "F.Cu") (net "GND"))
 (segment (start 185.415 102.835) (end 186 103.42) (width 0.2) (layer "F.Cu") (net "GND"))
 (segment (start 153.166346 83.858) (end 153.84 84.531654) (width 0.2) (layer "F.Cu") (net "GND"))
 (segment (start 167.7615 112.5085) (end 169.385 110.885) (width 0.2) (layer "F.Cu") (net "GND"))
 (segment (start 160.31 85.008) (end 159.16 83.858) (width 0.2) (layer "F.Cu") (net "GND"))
 (segment (start 160.490686 102.7035) (end 161.2035 102.7035) (width 0.2) (layer "F.Cu") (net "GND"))
 (segment (start 177.435 102.835) (end 169.385 110.885) (width 0.2) (layer "F.Cu") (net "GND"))
 (segment (start 177.435 102.835) (end 185.415 102.835) (width 0.2) (layer "F.Cu") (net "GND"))
 (segment (start 153.84 85.484346) (end 158.6635 90.307846) (width 0.2) (layer "F.Cu") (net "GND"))
 (segment (start 153.84 84.531654) (end 153.84 85.484346) (width 0.2) (layer "F.Cu") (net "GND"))
 (segment (start 135.235 118.095) (end 135.235 103.005) (width 0.2) (layer "F.Cu") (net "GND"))
 (segment (start 152.213654 83.858) (end 153.166346 83.858) (width 0.2) (layer "F.Cu") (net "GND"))
 (segment (start 158.6635 100.876314) (end 160.490686 102.7035) (width 0.2) (layer "F.Cu") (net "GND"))
 (segment (start 157.053654 83.858) (end 156.38 84.531654) (width 0.2) (layer "F.Cu") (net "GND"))
 (segment (start 135.235 100.836654) (end 152.213654 83.858) (width 0.2) (layer "F.Cu") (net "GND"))
 (segment (start 161.2035 102.7035) (end 169.385 110.885) (width 0.2) (layer "F.Cu") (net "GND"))
 (segment (start 161.2035 90.307846) (end 161.2035 102.7035) (width 0.2) (layer "F.Cu") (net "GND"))
 (segment (start 167.7615 116.455) (end 167.7615 112.5085) (width 0.2) (layer "F.Cu") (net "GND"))
 (segment (start 135.235 103.005) (end 135.235 100.836654) (width 0.2) (layer "F.Cu") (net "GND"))
 (segment (start 159.16 83.858) (end 157.053654 83.858) (width 0.2) (layer "F.Cu") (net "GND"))
 (segment (start 156.38 84.531654) (end 156.38 85.484346) (width 0.2) (layer "F.Cu") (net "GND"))
 (segment (start 158.6635 90.307846) (end 158.6635 100.876314) (width 0.2) (layer "F.Cu") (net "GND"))
 (segment (start 167.321605 101.442) (end 176.288 101.442) (width 0.2) (layer "F.Cu") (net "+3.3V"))
 (segment (start 189.49 107.01) (end 190.5 106) (width 0.2) (layer "F.Cu") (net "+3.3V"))
 (segment (start 185.99 107.01) (end 189.49 107.01) (width 0.2) (layer "F.Cu") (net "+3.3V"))
 (segment (start 184.95 109.99) (end 184.95 108.05) (width 0.2) (layer "F.Cu") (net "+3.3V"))
 (segment (start 184.95 108.05) (end 185.99 107.01) (width 0.2) (layer "F.Cu") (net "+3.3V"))
 (segment (start 166.6995 100.819895) (end 167.321605 101.442) (width 0.2) (layer "F.Cu") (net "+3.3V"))
 (segment (start 190.5 106) (end 190.5 101) (width 0.2) (layer "F.Cu") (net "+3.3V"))
 (segment (start 179.205 100.295) (end 177.435 100.295) (width 0.2) (layer "F.Cu") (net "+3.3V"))
 (segment (start 186 111.04) (end 184.95 109.99) (width 0.2) (layer "F.Cu") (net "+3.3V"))
 (segment (start 188.5 99) (end 180.5 99) (width 0.2) (layer "F.Cu") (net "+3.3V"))
 (segment (start 165.2215 116.455) (end 165.2215 123.1585) (width 0.2) (layer "F.Cu") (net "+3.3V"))
 (segment (start 180.5 99) (end 179.205 100.295) (width 0.2) (layer "F.Cu") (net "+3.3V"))
 (segment (start 165.2215 123.1585) (end 159.38 129) (width 0.2) (layer "F.Cu") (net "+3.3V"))
 (segment (start 157.77 85.008) (end 166.6995 93.9375) (width 0.2) (layer "F.Cu") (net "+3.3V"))
 (segment (start 176.288 101.442) (end 177.435 100.295) (width 0.2) (layer "F.Cu") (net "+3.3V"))
 (segment (start 190.5 101) (end 188.5 99) (width 0.2) (layer "F.Cu") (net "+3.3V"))
 (segment (start 166.6995 93.9375) (end 166.6995 100.819895) (width 0.2) (layer "F.Cu") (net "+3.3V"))
 (segment (start 181.5 129) (end 167 129) (width 0.2) (layer "F.Cu") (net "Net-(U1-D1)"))
 (segment (start 188.5 122) (end 181.5 129) (width 0.2) (layer "F.Cu") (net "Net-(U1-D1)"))
 (segment (start 188.5 111) (end 188.5 122) (width 0.2) (layer "F.Cu") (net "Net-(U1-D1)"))
 (segment (start 186 108.5) (end 189.5 108.5) (width 0.2) (layer "F.Cu") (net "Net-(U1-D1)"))
 (segment (start 186 108.5) (end 188.5 111) (width 0.2) (layer "F.Cu") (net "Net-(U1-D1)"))
 (segment (start 192.5 102) (end 188 97.5) (width 0.2) (layer "F.Cu") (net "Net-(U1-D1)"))
 (segment (start 189.5 108.5) (end 192.5 105.5) (width 0.2) (layer "F.Cu") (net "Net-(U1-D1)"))
 (segment (start 169.8065 97.5) (end 167.7615 99.545) (width 0.2) (layer "F.Cu") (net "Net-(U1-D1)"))
 (segment (start 188 97.5) (end 169.8065 97.5) (width 0.2) (layer "F.Cu") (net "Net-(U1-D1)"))
 (segment (start 192.5 105.5) (end 192.5 102) (width 0.2) (layer "F.Cu") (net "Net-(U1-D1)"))
 (segment (start 185.749925 101.685) (end 176.958654 101.685) (width 0.2) (layer "F.Cu") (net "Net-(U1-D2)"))
 (segment (start 176.958654 101.685) (end 176.801654 101.842) (width 0.2) (layer "F.Cu") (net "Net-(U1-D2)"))
 (segment (start 187.05 103.854925) (end 187.05 102.985075) (width 0.2) (layer "F.Cu") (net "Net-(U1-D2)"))
 (segment (start 158.965786 130) (end 159.794214 130) (width 0.2) (layer "F.Cu") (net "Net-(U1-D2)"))
 (segment (start 185.565075 104.47) (end 186.434925 104.47) (width 0.2) (layer "F.Cu") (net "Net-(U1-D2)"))
 (segment (start 187.05 102.985075) (end 185.749925 101.685) (width 0.2) (layer "F.Cu") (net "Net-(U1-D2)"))
 (segment (start 186.434925 104.47) (end 187.05 103.854925) (width 0.2) (layer "F.Cu") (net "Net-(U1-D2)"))
 (segment (start 141.585 100.465) (end 141.585 112.619214) (width 0.2) (layer "F.Cu") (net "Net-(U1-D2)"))
 (segment (start 175.9 110.123654) (end 176.958654 109.065) (width 0.2) (layer "F.Cu") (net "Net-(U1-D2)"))
 (segment (start 159.794214 130) (end 175.9 113.894214) (width 0.2) (layer "F.Cu") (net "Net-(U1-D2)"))
 (segment (start 175.9 113.894214) (end 175.9 110.123654) (width 0.2) (layer "F.Cu") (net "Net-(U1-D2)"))
 (segment (start 176.801654 101.842) (end 167.155919 101.842) (width 0.2) (layer "F.Cu") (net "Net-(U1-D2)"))
 (segment (start 180.970075 109.065) (end 185.565075 104.47) (width 0.2) (layer "F.Cu") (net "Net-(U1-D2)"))
 (segment (start 176.958654 109.065) (end 180.970075 109.065) (width 0.2) (layer "F.Cu") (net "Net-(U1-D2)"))
 (segment (start 165.2215 99.907581) (end 165.2215 99.545) (width 0.2) (layer "F.Cu") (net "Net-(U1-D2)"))
 (segment (start 141.585 112.619214) (end 158.965786 130) (width 0.2) (layer "F.Cu") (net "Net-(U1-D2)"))
 (segment (start 167.155919 101.842) (end 165.2215 99.907581) (width 0.2) (layer "F.Cu") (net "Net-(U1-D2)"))
 (segment (start 141.585 115.555) (end 136.695 110.665) (width 0.2) (layer "F.Cu") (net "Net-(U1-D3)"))
 (segment (start 159.679605 106.5) (end 160.5 106.5) (width 0.2) (layer "F.Cu") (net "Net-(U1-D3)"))
 (segment (start 152.244605 99.065) (end 159.679605 106.5) (width 0.2) (layer "F.Cu") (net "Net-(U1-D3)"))
 (segment (start 136.695 110.665) (end 136.695 103.375101) (width 0.2) (layer "F.Cu") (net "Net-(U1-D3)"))
 (segment (start 136.695 103.375101) (end 141.005101 99.065) (width 0.2) (layer "F.Cu") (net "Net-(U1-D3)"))
 (segment (start 141.005101 99.065) (end 152.244605 99.065) (width 0.2) (layer "F.Cu") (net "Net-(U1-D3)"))
 (via (at 160.5 106.5) (size 0.6) (drill 0.3) (layers "F.Cu" "B.Cu") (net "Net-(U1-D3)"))
 (segment (start 160.5 106.5) (end 162.6815 104.3185) (width 0.2) (layer "B.Cu") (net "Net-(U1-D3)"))
 (segment (start 162.6815 104.3185) (end 162.6815 100.38) (width 0.2) (layer "B.Cu") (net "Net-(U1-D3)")))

